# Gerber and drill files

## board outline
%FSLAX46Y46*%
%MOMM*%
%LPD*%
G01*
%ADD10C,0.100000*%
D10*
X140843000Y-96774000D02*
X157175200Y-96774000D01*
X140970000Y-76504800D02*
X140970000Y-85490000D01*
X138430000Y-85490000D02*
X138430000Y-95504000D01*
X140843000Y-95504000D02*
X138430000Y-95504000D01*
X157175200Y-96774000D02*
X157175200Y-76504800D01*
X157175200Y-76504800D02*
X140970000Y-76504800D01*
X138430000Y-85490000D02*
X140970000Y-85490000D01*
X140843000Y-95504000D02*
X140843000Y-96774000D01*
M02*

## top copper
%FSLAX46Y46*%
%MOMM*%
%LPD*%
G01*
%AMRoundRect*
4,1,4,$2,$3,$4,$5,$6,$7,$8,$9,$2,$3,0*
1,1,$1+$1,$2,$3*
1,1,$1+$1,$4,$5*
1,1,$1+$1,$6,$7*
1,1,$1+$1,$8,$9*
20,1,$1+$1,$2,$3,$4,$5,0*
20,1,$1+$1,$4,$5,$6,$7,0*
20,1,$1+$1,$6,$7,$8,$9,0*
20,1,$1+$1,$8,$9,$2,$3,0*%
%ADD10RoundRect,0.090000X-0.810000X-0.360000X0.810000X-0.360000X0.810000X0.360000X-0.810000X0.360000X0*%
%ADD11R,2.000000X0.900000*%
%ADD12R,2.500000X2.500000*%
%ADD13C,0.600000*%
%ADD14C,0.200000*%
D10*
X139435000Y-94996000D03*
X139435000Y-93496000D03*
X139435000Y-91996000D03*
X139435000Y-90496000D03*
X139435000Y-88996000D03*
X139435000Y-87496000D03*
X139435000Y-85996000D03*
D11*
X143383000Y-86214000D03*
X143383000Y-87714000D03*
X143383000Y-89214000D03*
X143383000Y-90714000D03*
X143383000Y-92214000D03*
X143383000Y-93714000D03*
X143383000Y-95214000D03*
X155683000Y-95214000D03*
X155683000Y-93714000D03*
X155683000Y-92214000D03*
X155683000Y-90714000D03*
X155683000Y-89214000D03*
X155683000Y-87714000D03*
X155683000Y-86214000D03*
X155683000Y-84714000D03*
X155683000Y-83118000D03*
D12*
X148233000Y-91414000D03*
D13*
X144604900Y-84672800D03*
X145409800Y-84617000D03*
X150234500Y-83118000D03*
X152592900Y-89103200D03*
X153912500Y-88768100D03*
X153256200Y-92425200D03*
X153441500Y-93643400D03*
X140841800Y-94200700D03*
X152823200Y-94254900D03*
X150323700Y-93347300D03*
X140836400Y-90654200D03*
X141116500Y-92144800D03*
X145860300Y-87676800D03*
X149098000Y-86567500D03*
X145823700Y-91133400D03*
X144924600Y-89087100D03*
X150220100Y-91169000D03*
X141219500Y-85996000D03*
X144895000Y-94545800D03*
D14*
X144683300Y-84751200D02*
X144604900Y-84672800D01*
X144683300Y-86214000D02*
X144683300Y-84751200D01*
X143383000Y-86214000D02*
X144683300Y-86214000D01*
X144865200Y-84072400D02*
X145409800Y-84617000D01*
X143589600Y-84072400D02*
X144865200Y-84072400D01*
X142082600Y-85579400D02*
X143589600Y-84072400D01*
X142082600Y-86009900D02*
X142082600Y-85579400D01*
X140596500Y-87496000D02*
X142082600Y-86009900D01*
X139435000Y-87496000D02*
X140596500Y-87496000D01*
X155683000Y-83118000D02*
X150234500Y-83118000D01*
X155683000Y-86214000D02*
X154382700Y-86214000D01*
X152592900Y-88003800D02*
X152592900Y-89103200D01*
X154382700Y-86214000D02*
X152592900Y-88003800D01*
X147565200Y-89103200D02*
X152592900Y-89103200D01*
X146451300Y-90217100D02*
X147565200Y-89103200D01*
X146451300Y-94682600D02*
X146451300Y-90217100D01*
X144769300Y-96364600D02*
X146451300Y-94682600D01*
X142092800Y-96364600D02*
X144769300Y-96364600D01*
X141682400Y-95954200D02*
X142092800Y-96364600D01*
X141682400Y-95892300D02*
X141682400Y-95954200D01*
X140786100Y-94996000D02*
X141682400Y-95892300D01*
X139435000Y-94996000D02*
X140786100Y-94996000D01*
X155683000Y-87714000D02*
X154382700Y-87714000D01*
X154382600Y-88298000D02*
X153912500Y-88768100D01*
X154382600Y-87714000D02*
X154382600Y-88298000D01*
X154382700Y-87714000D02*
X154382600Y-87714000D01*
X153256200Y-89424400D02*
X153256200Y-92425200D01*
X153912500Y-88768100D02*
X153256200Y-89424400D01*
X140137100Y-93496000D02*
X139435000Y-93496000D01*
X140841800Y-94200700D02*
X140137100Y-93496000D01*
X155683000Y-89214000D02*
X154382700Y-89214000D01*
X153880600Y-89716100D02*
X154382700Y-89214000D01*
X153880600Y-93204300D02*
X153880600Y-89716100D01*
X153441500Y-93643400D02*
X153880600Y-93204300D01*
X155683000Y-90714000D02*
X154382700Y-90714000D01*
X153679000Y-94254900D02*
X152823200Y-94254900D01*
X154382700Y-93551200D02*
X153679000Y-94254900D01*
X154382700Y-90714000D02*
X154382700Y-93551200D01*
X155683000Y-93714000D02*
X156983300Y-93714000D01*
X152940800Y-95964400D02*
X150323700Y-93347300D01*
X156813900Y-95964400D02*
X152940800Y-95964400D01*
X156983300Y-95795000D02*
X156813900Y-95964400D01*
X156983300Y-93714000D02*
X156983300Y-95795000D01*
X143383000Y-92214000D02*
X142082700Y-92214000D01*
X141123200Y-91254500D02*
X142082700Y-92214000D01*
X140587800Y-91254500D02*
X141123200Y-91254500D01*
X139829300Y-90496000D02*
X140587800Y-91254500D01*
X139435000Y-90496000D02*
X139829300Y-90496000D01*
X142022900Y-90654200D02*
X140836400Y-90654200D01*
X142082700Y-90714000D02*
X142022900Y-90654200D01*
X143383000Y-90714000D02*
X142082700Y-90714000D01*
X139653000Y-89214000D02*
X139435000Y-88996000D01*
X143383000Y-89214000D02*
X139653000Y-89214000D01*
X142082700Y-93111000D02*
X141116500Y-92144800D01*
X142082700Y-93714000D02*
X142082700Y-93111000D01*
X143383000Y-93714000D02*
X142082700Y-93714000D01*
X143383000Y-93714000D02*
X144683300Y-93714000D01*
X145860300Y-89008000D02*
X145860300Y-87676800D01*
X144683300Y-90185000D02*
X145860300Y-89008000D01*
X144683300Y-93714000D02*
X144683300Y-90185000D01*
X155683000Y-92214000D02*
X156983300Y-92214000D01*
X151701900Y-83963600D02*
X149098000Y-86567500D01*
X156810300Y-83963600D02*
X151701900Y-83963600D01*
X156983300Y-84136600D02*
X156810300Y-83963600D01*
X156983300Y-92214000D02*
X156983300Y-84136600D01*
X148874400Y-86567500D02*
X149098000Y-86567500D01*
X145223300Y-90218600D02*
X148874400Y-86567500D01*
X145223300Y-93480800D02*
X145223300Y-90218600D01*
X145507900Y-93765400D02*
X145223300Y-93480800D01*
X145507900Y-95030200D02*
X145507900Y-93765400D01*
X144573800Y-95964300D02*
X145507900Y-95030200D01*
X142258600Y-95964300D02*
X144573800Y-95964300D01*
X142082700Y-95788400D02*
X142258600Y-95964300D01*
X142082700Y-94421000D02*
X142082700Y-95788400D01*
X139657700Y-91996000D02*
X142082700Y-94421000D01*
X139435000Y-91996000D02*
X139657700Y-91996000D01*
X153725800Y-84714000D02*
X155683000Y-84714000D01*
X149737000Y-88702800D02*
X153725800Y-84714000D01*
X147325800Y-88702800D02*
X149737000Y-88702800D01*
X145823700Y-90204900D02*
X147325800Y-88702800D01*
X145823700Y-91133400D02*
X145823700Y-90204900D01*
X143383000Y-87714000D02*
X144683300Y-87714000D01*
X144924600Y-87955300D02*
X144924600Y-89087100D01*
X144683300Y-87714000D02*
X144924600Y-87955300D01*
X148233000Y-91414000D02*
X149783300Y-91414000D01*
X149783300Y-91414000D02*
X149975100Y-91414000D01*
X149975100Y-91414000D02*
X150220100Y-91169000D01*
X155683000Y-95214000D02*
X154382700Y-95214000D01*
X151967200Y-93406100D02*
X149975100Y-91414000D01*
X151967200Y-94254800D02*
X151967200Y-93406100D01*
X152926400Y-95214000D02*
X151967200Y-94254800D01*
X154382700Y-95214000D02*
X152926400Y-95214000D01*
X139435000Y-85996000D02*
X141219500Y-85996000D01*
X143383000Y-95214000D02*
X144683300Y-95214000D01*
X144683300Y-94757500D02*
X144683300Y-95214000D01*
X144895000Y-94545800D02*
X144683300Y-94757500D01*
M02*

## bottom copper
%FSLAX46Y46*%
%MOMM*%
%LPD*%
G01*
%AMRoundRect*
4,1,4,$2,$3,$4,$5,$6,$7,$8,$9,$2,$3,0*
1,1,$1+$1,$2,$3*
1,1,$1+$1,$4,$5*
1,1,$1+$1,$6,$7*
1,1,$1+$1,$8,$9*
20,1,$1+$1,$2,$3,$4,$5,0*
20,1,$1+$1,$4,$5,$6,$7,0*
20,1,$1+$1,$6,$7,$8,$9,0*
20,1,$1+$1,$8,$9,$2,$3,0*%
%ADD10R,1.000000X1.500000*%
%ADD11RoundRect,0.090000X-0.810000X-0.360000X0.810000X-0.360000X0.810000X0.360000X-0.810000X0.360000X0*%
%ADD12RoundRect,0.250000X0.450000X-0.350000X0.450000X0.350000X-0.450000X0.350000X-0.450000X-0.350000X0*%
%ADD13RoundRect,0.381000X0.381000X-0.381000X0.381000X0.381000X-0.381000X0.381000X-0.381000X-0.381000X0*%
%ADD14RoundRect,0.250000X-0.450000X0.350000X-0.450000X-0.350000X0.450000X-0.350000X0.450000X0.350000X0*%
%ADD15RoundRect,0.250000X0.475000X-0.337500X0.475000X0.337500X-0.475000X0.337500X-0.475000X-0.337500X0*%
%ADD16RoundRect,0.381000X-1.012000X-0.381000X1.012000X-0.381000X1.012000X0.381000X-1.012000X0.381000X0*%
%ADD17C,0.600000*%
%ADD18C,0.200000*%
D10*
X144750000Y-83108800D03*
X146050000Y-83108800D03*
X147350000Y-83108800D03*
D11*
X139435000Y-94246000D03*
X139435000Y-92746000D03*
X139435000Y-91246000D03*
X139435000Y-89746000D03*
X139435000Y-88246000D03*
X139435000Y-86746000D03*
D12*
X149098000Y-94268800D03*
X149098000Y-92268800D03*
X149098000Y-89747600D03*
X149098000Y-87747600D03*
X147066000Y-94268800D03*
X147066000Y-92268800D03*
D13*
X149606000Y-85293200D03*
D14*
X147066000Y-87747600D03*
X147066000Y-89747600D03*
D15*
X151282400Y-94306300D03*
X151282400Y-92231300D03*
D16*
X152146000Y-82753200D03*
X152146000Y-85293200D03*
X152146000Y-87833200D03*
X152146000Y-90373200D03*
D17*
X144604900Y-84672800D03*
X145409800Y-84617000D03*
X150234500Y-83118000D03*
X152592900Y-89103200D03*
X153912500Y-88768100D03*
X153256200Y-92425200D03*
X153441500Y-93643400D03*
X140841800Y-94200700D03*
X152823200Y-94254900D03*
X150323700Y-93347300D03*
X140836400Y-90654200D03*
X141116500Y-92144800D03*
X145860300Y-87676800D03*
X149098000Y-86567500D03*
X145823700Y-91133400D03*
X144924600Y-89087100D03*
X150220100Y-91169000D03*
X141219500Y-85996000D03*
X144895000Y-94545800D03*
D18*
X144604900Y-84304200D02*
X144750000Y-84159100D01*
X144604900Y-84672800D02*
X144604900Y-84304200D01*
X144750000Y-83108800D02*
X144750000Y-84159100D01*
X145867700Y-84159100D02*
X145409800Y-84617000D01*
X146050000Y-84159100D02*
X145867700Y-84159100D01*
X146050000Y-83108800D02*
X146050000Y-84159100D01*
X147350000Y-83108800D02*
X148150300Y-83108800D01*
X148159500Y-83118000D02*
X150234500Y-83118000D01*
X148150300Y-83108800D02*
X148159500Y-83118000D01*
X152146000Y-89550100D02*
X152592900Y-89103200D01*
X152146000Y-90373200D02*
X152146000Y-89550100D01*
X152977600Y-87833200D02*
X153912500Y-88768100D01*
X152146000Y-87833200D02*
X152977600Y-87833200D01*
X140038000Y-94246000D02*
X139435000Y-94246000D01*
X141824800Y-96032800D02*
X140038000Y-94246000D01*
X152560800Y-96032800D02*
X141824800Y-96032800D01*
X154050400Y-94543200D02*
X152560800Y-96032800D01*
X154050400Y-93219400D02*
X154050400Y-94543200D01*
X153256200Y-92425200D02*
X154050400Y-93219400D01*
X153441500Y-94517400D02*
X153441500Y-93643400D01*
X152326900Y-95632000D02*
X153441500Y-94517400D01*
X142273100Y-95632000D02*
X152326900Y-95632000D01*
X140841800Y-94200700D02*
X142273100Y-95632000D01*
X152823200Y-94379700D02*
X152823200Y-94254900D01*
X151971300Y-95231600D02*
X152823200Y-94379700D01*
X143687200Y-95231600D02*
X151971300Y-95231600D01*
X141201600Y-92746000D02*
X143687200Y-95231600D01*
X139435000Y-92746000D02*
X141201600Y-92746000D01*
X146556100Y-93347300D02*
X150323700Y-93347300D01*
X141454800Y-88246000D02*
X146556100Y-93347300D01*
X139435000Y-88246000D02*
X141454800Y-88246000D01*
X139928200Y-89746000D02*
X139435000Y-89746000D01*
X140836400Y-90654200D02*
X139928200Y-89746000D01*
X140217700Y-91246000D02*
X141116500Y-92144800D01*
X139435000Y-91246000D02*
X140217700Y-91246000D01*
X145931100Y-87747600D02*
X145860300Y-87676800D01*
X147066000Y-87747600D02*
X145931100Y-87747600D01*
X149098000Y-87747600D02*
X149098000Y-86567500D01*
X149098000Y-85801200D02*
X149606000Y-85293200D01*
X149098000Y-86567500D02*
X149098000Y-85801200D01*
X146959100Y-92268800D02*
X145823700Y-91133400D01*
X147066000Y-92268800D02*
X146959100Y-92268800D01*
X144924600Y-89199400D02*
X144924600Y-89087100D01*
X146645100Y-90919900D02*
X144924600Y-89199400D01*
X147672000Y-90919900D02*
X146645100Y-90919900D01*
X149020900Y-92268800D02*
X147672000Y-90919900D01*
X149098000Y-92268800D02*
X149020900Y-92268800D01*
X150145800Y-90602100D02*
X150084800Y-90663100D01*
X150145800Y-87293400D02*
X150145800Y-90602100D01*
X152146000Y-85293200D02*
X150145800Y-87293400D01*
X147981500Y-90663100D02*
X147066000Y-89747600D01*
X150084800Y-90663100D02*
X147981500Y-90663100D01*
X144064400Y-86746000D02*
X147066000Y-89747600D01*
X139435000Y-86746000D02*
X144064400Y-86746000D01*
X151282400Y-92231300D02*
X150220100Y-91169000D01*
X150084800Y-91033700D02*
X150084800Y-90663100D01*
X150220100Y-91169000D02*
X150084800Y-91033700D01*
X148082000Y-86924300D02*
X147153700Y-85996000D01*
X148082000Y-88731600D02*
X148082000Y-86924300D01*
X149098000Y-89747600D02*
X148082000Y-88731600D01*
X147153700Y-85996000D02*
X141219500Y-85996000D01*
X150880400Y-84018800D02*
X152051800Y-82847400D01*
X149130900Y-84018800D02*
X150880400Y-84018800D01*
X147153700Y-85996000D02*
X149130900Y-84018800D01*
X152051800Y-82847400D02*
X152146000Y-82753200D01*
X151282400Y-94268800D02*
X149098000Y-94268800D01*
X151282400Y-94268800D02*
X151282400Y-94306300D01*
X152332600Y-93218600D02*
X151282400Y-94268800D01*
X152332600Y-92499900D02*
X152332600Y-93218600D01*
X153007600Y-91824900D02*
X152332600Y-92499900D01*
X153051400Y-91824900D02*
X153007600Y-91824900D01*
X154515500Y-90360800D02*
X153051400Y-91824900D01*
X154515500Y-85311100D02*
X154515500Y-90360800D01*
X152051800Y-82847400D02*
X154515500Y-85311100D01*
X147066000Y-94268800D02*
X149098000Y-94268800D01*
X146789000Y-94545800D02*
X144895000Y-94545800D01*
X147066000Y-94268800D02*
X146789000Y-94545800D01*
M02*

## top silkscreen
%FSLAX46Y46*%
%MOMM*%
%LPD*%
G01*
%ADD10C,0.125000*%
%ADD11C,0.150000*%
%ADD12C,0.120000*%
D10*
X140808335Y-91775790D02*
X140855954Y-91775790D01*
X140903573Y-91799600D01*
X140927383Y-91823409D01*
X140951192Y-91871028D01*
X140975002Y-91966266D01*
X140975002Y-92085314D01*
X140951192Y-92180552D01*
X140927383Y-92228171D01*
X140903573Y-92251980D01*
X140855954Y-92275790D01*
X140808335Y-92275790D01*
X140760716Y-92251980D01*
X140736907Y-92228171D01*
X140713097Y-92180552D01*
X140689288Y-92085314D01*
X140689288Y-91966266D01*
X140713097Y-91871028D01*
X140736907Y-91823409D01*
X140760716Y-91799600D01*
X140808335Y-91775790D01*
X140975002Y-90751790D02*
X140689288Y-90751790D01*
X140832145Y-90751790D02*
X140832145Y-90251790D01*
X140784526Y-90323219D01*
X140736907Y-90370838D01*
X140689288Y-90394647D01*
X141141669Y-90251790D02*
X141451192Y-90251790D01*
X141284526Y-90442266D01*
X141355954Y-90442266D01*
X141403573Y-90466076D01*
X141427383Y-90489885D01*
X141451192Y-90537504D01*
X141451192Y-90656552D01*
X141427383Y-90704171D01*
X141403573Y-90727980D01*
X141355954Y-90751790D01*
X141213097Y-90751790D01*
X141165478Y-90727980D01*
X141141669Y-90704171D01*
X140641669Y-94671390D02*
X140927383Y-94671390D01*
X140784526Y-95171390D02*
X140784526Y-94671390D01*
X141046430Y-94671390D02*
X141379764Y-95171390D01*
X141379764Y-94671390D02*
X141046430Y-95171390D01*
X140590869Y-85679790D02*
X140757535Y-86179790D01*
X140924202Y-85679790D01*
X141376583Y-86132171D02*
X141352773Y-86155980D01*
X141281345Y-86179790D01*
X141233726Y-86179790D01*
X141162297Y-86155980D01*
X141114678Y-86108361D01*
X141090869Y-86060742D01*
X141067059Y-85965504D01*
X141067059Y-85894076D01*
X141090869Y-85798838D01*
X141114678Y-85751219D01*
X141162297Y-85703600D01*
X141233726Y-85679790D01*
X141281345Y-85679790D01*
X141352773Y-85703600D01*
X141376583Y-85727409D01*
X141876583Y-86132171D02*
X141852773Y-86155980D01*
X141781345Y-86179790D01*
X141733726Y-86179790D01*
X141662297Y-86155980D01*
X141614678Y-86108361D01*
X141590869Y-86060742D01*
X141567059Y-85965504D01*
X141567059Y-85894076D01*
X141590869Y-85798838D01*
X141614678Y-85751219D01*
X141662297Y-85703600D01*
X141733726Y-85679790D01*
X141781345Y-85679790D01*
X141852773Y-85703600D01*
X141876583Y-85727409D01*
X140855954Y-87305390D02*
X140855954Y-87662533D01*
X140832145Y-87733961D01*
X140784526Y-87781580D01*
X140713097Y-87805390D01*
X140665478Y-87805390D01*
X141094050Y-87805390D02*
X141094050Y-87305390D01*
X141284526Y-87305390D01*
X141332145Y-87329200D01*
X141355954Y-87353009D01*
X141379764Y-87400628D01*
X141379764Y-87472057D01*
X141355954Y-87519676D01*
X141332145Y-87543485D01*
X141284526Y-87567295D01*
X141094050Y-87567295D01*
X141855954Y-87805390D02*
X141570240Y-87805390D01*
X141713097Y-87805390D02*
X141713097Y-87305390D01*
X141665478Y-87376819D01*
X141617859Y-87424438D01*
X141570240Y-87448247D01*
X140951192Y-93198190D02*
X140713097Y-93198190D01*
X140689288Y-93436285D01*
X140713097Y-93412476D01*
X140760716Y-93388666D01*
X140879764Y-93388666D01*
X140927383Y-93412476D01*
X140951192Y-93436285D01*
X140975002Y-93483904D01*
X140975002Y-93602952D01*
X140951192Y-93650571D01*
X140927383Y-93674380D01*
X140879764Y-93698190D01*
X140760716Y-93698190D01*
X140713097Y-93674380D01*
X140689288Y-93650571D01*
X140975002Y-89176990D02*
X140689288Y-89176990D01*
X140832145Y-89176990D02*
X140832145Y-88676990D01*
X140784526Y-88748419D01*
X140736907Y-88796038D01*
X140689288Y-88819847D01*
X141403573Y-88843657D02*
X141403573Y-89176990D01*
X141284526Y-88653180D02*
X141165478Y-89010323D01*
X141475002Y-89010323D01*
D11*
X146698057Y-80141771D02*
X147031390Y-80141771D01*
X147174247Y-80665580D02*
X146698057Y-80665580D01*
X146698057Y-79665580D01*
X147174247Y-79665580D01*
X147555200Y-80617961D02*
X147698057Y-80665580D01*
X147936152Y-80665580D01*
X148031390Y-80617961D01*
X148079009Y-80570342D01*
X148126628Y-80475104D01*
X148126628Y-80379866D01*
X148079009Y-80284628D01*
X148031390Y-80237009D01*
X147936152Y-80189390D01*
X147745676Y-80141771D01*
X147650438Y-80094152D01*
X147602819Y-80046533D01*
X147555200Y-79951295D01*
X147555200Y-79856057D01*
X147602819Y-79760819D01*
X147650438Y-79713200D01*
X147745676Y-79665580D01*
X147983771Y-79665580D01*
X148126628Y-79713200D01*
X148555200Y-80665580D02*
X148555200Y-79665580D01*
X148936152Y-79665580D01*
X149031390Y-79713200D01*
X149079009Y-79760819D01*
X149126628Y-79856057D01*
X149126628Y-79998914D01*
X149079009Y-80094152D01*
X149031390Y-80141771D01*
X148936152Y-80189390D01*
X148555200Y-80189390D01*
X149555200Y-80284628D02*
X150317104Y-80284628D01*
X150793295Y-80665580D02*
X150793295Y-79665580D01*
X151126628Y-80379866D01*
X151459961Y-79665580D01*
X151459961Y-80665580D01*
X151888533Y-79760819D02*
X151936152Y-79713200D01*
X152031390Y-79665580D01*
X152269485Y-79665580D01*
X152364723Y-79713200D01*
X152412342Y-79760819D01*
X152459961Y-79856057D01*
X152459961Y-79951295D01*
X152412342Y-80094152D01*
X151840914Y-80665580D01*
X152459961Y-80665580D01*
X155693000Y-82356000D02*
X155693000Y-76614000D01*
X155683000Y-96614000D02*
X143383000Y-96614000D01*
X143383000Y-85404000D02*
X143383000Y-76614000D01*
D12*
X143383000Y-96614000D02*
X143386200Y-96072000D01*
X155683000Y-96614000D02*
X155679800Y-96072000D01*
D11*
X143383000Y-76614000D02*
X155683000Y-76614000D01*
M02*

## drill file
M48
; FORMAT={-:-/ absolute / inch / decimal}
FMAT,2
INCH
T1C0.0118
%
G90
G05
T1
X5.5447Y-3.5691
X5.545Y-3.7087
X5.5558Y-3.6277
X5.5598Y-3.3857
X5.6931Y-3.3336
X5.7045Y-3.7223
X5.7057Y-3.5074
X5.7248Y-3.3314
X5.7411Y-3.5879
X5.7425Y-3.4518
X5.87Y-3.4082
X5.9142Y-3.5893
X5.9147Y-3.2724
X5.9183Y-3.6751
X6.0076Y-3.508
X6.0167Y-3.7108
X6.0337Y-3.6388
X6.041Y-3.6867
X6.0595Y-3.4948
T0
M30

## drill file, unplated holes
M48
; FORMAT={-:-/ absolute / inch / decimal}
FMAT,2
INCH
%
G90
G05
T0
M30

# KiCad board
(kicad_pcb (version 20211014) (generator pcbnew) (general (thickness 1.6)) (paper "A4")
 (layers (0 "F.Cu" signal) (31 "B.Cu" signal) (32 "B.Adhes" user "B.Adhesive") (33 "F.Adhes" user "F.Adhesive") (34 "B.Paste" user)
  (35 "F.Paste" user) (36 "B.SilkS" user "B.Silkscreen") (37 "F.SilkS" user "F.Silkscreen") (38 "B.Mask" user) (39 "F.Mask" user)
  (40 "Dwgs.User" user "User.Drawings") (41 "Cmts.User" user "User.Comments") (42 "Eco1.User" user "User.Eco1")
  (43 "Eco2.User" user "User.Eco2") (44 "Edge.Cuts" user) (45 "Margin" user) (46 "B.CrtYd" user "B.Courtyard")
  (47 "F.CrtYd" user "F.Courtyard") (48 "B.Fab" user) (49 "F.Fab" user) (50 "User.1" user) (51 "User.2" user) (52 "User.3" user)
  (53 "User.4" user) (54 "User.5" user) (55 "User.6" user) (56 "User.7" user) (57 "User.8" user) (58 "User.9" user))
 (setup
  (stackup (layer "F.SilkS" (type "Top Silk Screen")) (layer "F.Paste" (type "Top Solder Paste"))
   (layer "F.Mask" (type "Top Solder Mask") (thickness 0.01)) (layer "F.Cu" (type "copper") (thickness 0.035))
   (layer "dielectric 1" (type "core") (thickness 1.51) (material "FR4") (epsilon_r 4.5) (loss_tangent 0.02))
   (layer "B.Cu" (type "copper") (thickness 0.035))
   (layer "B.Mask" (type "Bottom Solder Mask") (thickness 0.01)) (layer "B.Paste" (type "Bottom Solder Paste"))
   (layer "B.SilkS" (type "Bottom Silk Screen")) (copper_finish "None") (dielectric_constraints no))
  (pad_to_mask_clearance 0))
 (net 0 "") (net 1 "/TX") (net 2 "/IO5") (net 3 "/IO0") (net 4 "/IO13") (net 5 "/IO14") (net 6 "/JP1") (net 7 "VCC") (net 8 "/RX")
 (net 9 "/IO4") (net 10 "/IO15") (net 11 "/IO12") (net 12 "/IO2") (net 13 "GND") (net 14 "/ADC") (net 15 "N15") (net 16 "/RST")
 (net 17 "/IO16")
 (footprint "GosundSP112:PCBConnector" (layer "F.Cu") (at 140.335 94.996)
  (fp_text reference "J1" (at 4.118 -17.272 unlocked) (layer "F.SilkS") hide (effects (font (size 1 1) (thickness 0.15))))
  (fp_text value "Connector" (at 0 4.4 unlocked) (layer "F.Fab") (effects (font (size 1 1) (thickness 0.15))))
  (pad "1" smd roundrect (at -0.9 0) (size 1.8 0.9) (layers "F.Cu" "F.Paste" "F.Mask") (roundrect_rratio 0.1) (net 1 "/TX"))
  (pad "2" smd roundrect (at -0.9 -1.5) (size 1.8 0.9) (layers "F.Cu" "F.Paste" "F.Mask") (roundrect_rratio 0.1) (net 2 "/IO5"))
  (pad "3" smd roundrect (at -0.9 -3) (size 1.8 0.9) (layers "F.Cu" "F.Paste" "F.Mask") (roundrect_rratio 0.1) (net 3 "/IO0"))
  (pad "4" smd roundrect (at -0.9 -4.5) (size 1.8 0.9) (layers "F.Cu" "F.Paste" "F.Mask") (roundrect_rratio 0.1) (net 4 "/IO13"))
  (pad "5" smd roundrect (at -0.9 -6) (size 1.8 0.9) (layers "F.Cu" "F.Paste" "F.Mask") (roundrect_rratio 0.1) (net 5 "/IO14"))
  (pad "6" smd roundrect (at -0.9 -7.5) (size 1.8 0.9) (layers "F.Cu" "F.Paste" "F.Mask") (roundrect_rratio 0.1) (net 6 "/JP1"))
  (pad "7" smd roundrect (at -0.9 -9) (size 1.8 0.9) (layers "F.Cu" "F.Paste" "F.Mask") (roundrect_rratio 0.1) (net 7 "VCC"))
  (pad "8" smd roundrect (at -0.9 -0.75) (size 1.8 0.9) (layers "B.Cu" "B.Paste" "B.Mask") (roundrect_rratio 0.1) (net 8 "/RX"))
  (pad "9" smd roundrect (at -0.9 -2.25) (size 1.8 0.9) (layers "B.Cu" "B.Paste" "B.Mask") (roundrect_rratio 0.1) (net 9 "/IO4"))
  (pad "10" smd roundrect (at -0.9 -3.75) (size 1.8 0.9) (layers "B.Cu" "B.Paste" "B.Mask") (roundrect_rratio 0.1) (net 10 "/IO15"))
  (pad "11" smd roundrect (at -0.9 -5.25) (size 1.8 0.9) (layers "B.Cu" "B.Paste" "B.Mask") (roundrect_rratio 0.1) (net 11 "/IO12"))
  (pad "12" smd roundrect (at -0.9 -6.75) (size 1.8 0.9) (layers "B.Cu" "B.Paste" "B.Mask") (roundrect_rratio 0.1) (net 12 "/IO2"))
  (pad "13" smd roundrect (at -0.9 -8.25) (size 1.8 0.9) (layers "B.Cu" "B.Paste" "B.Mask") (roundrect_rratio 0.1) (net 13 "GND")))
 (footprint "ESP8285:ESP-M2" (layer "F.Cu") (at 149.533 89.214)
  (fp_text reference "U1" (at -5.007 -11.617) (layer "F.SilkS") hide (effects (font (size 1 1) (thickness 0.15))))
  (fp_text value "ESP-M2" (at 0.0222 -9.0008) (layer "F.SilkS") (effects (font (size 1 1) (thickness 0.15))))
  (fp_line (start 6.16 -6.858) (end 6.16 -12.6) (layer "F.SilkS") (width 0.15))
  (fp_line (start 6.15 7.4) (end -6.15 7.4) (layer "F.SilkS") (width 0.15))
  (fp_line (start -6.15 -3.81) (end -6.15 -12.6) (layer "F.SilkS") (width 0.15))
  (fp_line (start -6.15 7.4) (end -6.1468 6.858) (layer "F.SilkS") (width 0.12))
  (fp_line (start 6.15 7.4) (end 6.1468 6.858) (layer "F.SilkS") (width 0.12))
  (fp_line (start -6.15 -12.6) (end 6.15 -12.6) (layer "F.SilkS") (width 0.15))
  (pad "1" smd rect (at -6.15 -3 90) (size 0.9 2) (layers "F.Cu" "F.Paste" "F.Mask") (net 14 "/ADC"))
  (pad "2" smd rect (at -6.15 -1.5 90) (size 0.9 2) (layers "F.Cu" "F.Paste" "F.Mask") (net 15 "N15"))
  (pad "3" smd rect (at -6.15 0 90) (size 0.9 2) (layers "F.Cu" "F.Paste" "F.Mask") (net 5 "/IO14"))
  (pad "4" smd rect (at -6.15 1.5 90) (size 0.9 2) (layers "F.Cu" "F.Paste" "F.Mask") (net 11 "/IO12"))
  (pad "5" smd rect (at -6.15 3 90) (size 0.9 2) (layers "F.Cu" "F.Paste" "F.Mask") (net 4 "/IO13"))
  (pad "6" smd rect (at -6.15 4.5 90) (size 0.9 2) (layers "F.Cu" "F.Paste" "F.Mask") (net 10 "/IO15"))
  (pad "7" smd rect (at -6.15 6 90) (size 0.9 2) (layers "F.Cu" "F.Paste" "F.Mask") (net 7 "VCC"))
  (pad "8" smd rect (at 6.15 6 90) (size 0.9 2) (layers "F.Cu" "F.Paste" "F.Mask") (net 13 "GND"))
  (pad "9" smd rect (at 6.15 4.5 90) (size 0.9 2) (layers "F.Cu" "F.Paste" "F.Mask") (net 12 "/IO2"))
  (pad "10" smd rect (at 6.15 3 90) (size 0.9 2) (layers "F.Cu" "F.Paste" "F.Mask") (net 3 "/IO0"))
  (pad "11" smd rect (at 6.15 1.5 90) (size 0.9 2) (layers "F.Cu" "F.Paste" "F.Mask") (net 9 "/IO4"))
  (pad "12" smd rect (at 6.15 0 90) (size 0.9 2) (layers "F.Cu" "F.Paste" "F.Mask") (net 2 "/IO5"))
  (pad "13" smd rect (at 6.15 -1.5 90) (size 0.9 2) (layers "F.Cu" "F.Paste" "F.Mask") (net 8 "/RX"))
  (pad "14" smd rect (at 6.15 -3 90) (size 0.9 2) (layers "F.Cu" "F.Paste" "F.Mask") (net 1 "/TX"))
  (pad "15" smd rect (at 6.15 -4.5 90) (size 0.9 2) (layers "F.Cu" "F.Paste" "F.Mask") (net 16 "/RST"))
  (pad "16" smd rect (at 6.15 -6.096 90) (size 0.9 2) (layers "F.Cu" "F.Paste" "F.Mask") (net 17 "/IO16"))
  (pad "17" smd rect (at -1.3 2.2 90) (size 2.5 2.5) (layers "F.Cu" "F.Paste" "F.Mask") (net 13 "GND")))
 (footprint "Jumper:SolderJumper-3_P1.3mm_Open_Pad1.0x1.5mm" (layer "B.Cu") (at 146.05 83.1088)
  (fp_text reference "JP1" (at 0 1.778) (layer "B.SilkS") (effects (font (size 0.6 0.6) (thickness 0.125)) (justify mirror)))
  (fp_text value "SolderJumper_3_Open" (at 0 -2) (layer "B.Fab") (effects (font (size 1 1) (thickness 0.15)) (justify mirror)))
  (pad "1" smd rect (at -1.3 0) (size 1 1.5) (layers "B.Cu" "B.Mask") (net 14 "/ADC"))
  (pad "2" smd rect (at 0 0) (size 1 1.5) (layers "B.Cu" "B.Mask") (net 6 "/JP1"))
  (pad "3" smd rect (at 1.3 0) (size 1 1.5) (layers "B.Cu" "B.Mask") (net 17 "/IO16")))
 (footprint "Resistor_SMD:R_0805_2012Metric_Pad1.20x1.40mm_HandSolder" (layer "B.Cu") (at 149.098 93.2688 90)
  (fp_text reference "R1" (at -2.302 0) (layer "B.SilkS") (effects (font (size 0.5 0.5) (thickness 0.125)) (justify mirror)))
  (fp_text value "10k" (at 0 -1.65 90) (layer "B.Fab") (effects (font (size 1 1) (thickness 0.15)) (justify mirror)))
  (pad "1" smd roundrect (at -1 0 90) (size 1.2 1.4) (layers "B.Cu" "B.Paste" "B.Mask") (roundrect_rratio 0.2083333333) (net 7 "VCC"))
  (pad "2" smd roundrect (at 1 0 90) (size 1.2 1.4) (layers "B.Cu" "B.Paste" "B.Mask") (roundrect_rratio 0.2083333333) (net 15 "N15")))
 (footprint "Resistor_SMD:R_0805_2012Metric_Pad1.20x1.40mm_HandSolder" (layer "B.Cu") (at 149.098 88.7476 90)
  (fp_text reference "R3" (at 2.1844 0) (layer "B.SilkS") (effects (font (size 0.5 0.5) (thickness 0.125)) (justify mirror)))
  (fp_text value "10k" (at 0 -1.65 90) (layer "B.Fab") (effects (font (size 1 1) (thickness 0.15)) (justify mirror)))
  (pad "1" smd roundrect (at -1 0 90) (size 1.2 1.4) (layers "B.Cu" "B.Paste" "B.Mask") (roundrect_rratio 0.2083333333) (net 7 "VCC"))
  (pad "2" smd roundrect (at 1 0 90) (size 1.2 1.4) (layers "B.Cu" "B.Paste" "B.Mask") (roundrect_rratio 0.2083333333) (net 3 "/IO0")))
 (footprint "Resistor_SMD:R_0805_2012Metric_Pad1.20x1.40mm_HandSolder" (layer "B.Cu") (at 147.066 93.2688 90)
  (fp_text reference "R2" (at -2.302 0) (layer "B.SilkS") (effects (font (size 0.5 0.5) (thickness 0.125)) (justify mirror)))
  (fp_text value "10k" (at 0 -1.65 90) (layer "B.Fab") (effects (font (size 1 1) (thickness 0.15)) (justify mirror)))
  (pad "1" smd roundrect (at -1 0 90) (size 1.2 1.4) (layers "B.Cu" "B.Paste" "B.Mask") (roundrect_rratio 0.2083333333) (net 7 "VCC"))
  (pad "2" smd roundrect (at 1 0 90) (size 1.2 1.4) (layers "B.Cu" "B.Paste" "B.Mask") (roundrect_rratio 0.2083333333) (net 16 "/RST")))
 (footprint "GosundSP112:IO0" (layer "B.Cu") (at 147.066 85.2932 90)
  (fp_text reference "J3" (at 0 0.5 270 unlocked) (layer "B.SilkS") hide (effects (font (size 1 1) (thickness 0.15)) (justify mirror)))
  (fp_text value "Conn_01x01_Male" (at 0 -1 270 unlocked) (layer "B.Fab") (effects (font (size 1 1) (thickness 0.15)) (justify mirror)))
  (pad "1" smd roundrect (at 0 2.54 90) (size 1.524 1.524) (layers "B.Cu" "B.Paste" "B.Mask") (roundrect_rratio 0.25) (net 3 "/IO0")))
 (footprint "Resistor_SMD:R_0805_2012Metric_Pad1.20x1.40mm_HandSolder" (layer "B.Cu") (at 147.066 88.7476 -90)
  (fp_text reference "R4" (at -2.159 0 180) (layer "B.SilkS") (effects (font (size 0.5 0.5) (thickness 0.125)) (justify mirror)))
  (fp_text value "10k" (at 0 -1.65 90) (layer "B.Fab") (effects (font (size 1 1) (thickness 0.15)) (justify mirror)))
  (pad "1" smd roundrect (at -1 0 270) (size 1.2 1.4) (layers "B.Cu" "B.Paste" "B.Mask") (roundrect_rratio 0.2083333333) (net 10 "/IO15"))
  (pad "2" smd roundrect (at 1 0 270) (size 1.2 1.4) (layers "B.Cu" "B.Paste" "B.Mask") (roundrect_rratio 0.2083333333) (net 13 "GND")))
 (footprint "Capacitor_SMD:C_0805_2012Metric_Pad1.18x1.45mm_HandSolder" (layer "B.Cu") (at 151.2824 93.2688 90)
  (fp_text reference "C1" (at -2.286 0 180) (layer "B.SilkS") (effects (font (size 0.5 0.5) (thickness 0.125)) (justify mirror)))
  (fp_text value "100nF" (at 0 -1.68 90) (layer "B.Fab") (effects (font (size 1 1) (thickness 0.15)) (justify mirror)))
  (pad "1" smd roundrect (at -1.0375 0 90) (size 1.175 1.45) (layers "B.Cu" "B.Paste" "B.Mask") (roundrect_rratio 0.2127659574)
   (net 7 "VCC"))
  (pad "2" smd roundrect (at 1.0375 0 90) (size 1.175 1.45) (layers "B.Cu" "B.Paste" "B.Mask") (roundrect_rratio 0.2127659574)
   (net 13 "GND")))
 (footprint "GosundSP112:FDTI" (layer "B.Cu") (at 152.146 82.7532)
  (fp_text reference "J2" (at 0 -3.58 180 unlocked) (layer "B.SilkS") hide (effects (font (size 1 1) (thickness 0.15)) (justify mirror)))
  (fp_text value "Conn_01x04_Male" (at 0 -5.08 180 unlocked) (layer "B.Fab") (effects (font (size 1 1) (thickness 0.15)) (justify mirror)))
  (pad "1" smd roundrect (at 0 0) (size 2.786 1.524) (layers "B.Cu" "B.Paste" "B.Mask") (roundrect_rratio 0.25) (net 7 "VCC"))
  (pad "2" smd roundrect (at 0 2.54) (size 2.786 1.524) (layers "B.Cu" "B.Paste" "B.Mask") (roundrect_rratio 0.25) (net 13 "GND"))
  (pad "3" smd roundrect (at 0 5.08) (size 2.786 1.524) (layers "B.Cu" "B.Paste" "B.Mask") (roundrect_rratio 0.25) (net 8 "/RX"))
  (pad "4" smd roundrect (at 0 7.62) (size 2.786 1.524) (layers "B.Cu" "B.Paste" "B.Mask") (roundrect_rratio 0.25) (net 1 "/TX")))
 (gr_line (start 140.843 96.774) (end 157.1752 96.774) (layer "Edge.Cuts") (width 0.1))
 (gr_line (start 140.97 76.5048) (end 140.97 85.49) (layer "Edge.Cuts") (width 0.1))
 (gr_line (start 138.43 85.49) (end 138.43 95.504) (layer "Edge.Cuts") (width 0.1))
 (gr_line (start 140.843 95.504) (end 138.43 95.504) (layer "Edge.Cuts") (width 0.1))
 (gr_line (start 157.1752 96.774) (end 157.1752 76.5048) (layer "Edge.Cuts") (width 0.1))
 (gr_line (start 157.1752 76.5048) (end 140.97 76.5048) (layer "Edge.Cuts") (width 0.1))
 (gr_line (start 138.43 85.49) (end 140.97 85.49) (layer "Edge.Cuts") (width 0.1))
 (gr_line (start 140.843 95.504) (end 140.843 96.774) (layer "Edge.Cuts") (width 0.1))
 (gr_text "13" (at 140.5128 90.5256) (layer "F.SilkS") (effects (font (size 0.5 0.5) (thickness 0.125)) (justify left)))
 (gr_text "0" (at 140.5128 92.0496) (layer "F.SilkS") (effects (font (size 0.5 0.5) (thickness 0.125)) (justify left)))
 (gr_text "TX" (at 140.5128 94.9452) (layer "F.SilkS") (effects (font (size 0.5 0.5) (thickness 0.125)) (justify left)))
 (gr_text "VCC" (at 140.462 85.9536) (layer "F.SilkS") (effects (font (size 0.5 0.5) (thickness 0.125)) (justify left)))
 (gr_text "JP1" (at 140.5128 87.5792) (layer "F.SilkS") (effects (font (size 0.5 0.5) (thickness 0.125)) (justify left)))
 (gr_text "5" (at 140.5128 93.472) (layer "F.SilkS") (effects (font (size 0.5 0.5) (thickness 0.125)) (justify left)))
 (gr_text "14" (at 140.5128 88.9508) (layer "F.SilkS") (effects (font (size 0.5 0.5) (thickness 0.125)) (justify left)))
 (segment (start 144.6833 94.7575) (end 144.6833 95.214) (width 0.2) (layer "F.Cu") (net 7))
 (segment (start 143.383 95.214) (end 144.6833 95.214) (width 0.2) (layer "F.Cu") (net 7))
 (segment (start 144.895 94.5458) (end 144.6833 94.7575) (width 0.2) (layer "F.Cu") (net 7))
 (segment (start 139.435 85.996) (end 141.2195 85.996) (width 0.2) (layer "F.Cu") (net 7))
 (via (at 144.895 94.5458) (size 0.6) (drill 0.3) (layers "F.Cu" "B.Cu") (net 7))
 (via (at 141.2195 85.996) (size 0.6) (drill 0.3) (layers "F.Cu" "B.Cu") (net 7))
 (segment (start 152.3326 92.4999) (end 152.3326 93.2186) (width 0.2) (layer "B.Cu") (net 7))
 (segment (start 150.8804 84.0188) (end 152.0518 82.8474) (width 0.2) (layer "B.Cu") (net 7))
 (segment (start 147.066 94.2688) (end 149.098 94.2688) (width 0.2) (layer "B.Cu") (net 7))
 (segment (start 153.0514 91.8249) (end 153.0076 91.8249) (width 0.2) (layer "B.Cu") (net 7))
 (segment (start 147.1537 85.996) (end 141.2195 85.996) (width 0.2) (layer "B.Cu") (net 7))
 (segment (start 151.2824 94.2688) (end 149.098 94.2688) (width 0.2) (layer "B.Cu") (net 7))
 (segment (start 148.082 88.7316) (end 148.082 86.9243) (width 0.2) (layer "B.Cu") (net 7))
 (segment (start 146.789 94.5458) (end 144.895 94.5458) (width 0.2) (layer "B.Cu") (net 7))
 (segment (start 147.066 94.2688) (end 146.789 94.5458) (width 0.2) (layer "B.Cu") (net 7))
 (segment (start 152.0518 82.8474) (end 154.5155 85.3111) (width 0.2) (layer "B.Cu") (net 7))
 (segment (start 152.3326 93.2186) (end 151.2824 94.2688) (width 0.2) (layer "B.Cu") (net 7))
 (segment (start 153.0076 91.8249) (end 152.3326 92.4999) (width 0.2) (layer "B.Cu") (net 7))
 (segment (start 148.082 86.9243) (end 147.1537 85.996) (width 0.2) (layer "B.Cu") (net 7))
 (segment (start 147.1537 85.996) (end 149.1309 84.0188) (width 0.2) (layer "B.Cu") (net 7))
 (segment (start 149.1309 84.0188) (end 150.8804 84.0188) (width 0.2) (layer "B.Cu") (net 7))
 (segment (start 149.098 89.7476) (end 148.082 88.7316) (width 0.2) (layer "B.Cu") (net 7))
 (segment (start 152.0518 82.8474) (end 152.146 82.7532) (width 0.2) (layer "B.Cu") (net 7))
 (segment (start 151.2824 94.2688) (end 151.2824 94.3063) (width 0.2) (layer "B.Cu") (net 7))
 (segment (start 154.5155 85.3111) (end 154.5155 90.3608) (width 0.2) (layer "B.Cu") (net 7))
 (segment (start 154.5155 90.3608) (end 153.0514 91.8249) (width 0.2) (layer "B.Cu") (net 7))
 (segment (start 149.7833 91.414) (end 149.9751 91.414) (width 0.2) (layer "F.Cu") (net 13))
 (segment (start 149.9751 91.414) (end 150.2201 91.169) (width 0.2) (layer "F.Cu") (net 13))
 (segment (start 154.3827 95.214) (end 152.9264 95.214) (width 0.2) (layer "F.Cu") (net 13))
 (segment (start 152.9264 95.214) (end 151.9672 94.2548) (width 0.2) (layer "F.Cu") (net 13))
 (segment (start 151.9672 94.2548) (end 151.9672 93.4061) (width 0.2) (layer "F.Cu") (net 13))
 (segment (start 155.683 95.214) (end 154.3827 95.214) (width 0.2) (layer "F.Cu") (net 13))
 (segment (start 151.9672 93.4061) (end 149.9751 91.414) (width 0.2) (layer "F.Cu") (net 13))
 (segment (start 148.233 91.414) (end 149.7833 91.414) (width 0.2) (layer "F.Cu") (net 13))
 (via (at 150.2201 91.169) (size 0.6) (drill 0.3) (layers "F.Cu" "B.Cu") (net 13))
 (segment (start 150.0848 91.0337) (end 150.0848 90.6631) (width 0.2) (layer "B.Cu") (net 13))
 (segment (start 150.0848 90.6631) (end 147.9815 90.6631) (width 0.2) (layer "B.Cu") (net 13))
 (segment (start 144.0644 86.746) (end 147.066 89.7476) (width 0.2) (layer "B.Cu") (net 13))
 (segment (start 150.1458 87.2934) (end 150.1458 90.6021) (width 0.2) (layer "B.Cu") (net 13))
 (segment (start 147.9815 90.6631) (end 147.066 89.7476) (width 0.2) (layer "B.Cu") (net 13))
 (segment (start 150.2201 91.169) (end 150.0848 91.0337) (width 0.2) (layer "B.Cu") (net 13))
 (segment (start 152.146 85.2932) (end 150.1458 87.2934) (width 0.2) (layer "B.Cu") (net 13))
 (segment (start 151.2824 92.2313) (end 150.2201 91.169) (width 0.2) (layer "B.Cu") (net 13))
 (segment (start 139.435 86.746) (end 144.0644 86.746) (width 0.2) (layer "B.Cu") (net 13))
 (segment (start 150.1458 90.6021) (end 150.0848 90.6631) (width 0.2) (layer "B.Cu") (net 13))
 (segment (start 144.6833 87.714) (end 144.9246 87.9553) (width 0.2) (layer "F.Cu") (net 15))
 (segment (start 143.383 87.714) (end 144.6833 87.714) (width 0.2) (layer "F.Cu") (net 15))
 (segment (start 144.9246 87.9553) (end 144.9246 89.0871) (width 0.2) (layer "F.Cu") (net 15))
 (via (at 144.9246 89.0871) (size 0.6) (drill 0.3) (layers "F.Cu" "B.Cu") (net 15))
 (segment (start 147.672 90.9199) (end 146.6451 90.9199) (width 0.2) (layer "B.Cu") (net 15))
 (segment (start 149.098 92.2688) (end 149.0209 92.2688) (width 0.2) (layer "B.Cu") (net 15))
 (segment (start 149.0209 92.2688) (end 147.672 90.9199) (width 0.2) (layer "B.Cu") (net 15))
 (segment (start 146.6451 90.9199) (end 144.9246 89.1994) (width 0.2) (layer "B.Cu") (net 15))
 (segment (start 144.9246 89.1994) (end 144.9246 89.0871) (width 0.2) (layer "B.Cu") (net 15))
 (segment (start 145.8237 91.1334) (end 145.8237 90.2049) (width 0.2) (layer "F.Cu") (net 16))
 (segment (start 147.3258 88.7028) (end 149.737 88.7028) (width 0.2) (layer "F.Cu") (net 16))
 (segment (start 145.8237 90.2049) (end 147.3258 88.7028) (width 0.2) (layer "F.Cu") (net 16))
 (segment (start 153.7258 84.714) (end 155.683 84.714) (width 0.2) (layer "F.Cu") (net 16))
 (segment (start 149.737 88.7028) (end 153.7258 84.714) (width 0.2) (layer "F.Cu") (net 16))
 (via (at 145.8237 91.1334) (size 0.6) (drill 0.3) (layers "F.Cu" "B.Cu") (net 16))
 (segment (start 147.066 92.2688) (end 146.9591 92.2688) (width 0.2) (layer "B.Cu") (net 16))
 (segment (start 146.9591 92.2688) (end 145.8237 91.1334) (width 0.2) (layer "B.Cu") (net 16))
 (segment (start 156.9833 84.1366) (end 156.8103 83.9636) (width 0.2) (layer "F.Cu") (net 3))
 (segment (start 142.0827 95.7884) (end 142.2586 95.9643) (width 0.2) (layer "F.Cu") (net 3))
 (segment (start 145.2233 90.2186) (end 148.8744 86.5675) (width 0.2) (layer "F.Cu") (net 3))
 (segment (start 151.7019 83.9636) (end 149.098 86.5675) (width 0.2) (layer "F.Cu") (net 3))
 (segment (start 145.2233 93.4808) (end 145.2233 90.2186) (width 0.2) (layer "F.Cu") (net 3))
 (segment (start 156.9833 92.214) (end 156.9833 84.1366) (width 0.2) (layer "F.Cu") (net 3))
 (segment (start 155.683 92.214) (end 156.9833 92.214) (width 0.2) (layer "F.Cu") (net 3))
 (segment (start 142.0827 94.421) (end 142.0827 95.7884) (width 0.2) (layer "F.Cu") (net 3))
 (segment (start 142.2586 95.9643) (end 144.5738 95.9643) (width 0.2) (layer "F.Cu") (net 3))
 (segment (start 148.8744 86.5675) (end 149.098 86.5675) (width 0.2) (layer "F.Cu") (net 3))
 (segment (start 139.435 91.996) (end 139.6577 91.996) (width 0.2) (layer "F.Cu") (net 3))
 (segment (start 139.6577 91.996) (end 142.0827 94.421) (width 0.2) (layer "F.Cu") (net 3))
 (segment (start 145.5079 95.0302) (end 145.5079 93.7654) (width 0.2) (layer "F.Cu") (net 3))
 (segment (start 145.5079 93.7654) (end 145.2233 93.4808) (width 0.2) (layer "F.Cu") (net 3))
 (segment (start 156.8103 83.9636) (end 151.7019 83.9636) (width 0.2) (layer "F.Cu") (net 3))
 (segment (start 144.5738 95.9643) (end 145.5079 95.0302) (width 0.2) (layer "F.Cu") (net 3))
 (via (at 149.098 86.5675) (size 0.6) (drill 0.3) (layers "F.Cu" "B.Cu") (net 3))
 (segment (start 149.098 87.7476) (end 149.098 86.5675) (width 0.2) (layer "B.Cu") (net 3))
 (segment (start 149.098 86.5675) (end 149.098 85.8012) (width 0.2) (layer "B.Cu") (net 3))
 (segment (start 149.098 85.8012) (end 149.606 85.2932) (width 0.2) (layer "B.Cu") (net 3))
 (segment (start 144.6833 90.185) (end 145.8603 89.008) (width 0.2) (layer "F.Cu") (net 10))
 (segment (start 143.383 93.714) (end 142.0827 93.714) (width 0.2) (layer "F.Cu") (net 10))
 (segment (start 144.6833 93.714) (end 144.6833 90.185) (width 0.2) (layer "F.Cu") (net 10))
 (segment (start 142.0827 93.714) (end 142.0827 93.111) (width 0.2) (layer "F.Cu") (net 10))
 (segment (start 142.0827 93.111) (end 141.1165 92.1448) (width 0.2) (layer "F.Cu") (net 10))
 (segment (start 145.8603 89.008) (end 145.8603 87.6768) (width 0.2) (layer "F.Cu") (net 10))
 (segment (start 143.383 93.714) (end 144.6833 93.714) (width 0.2) (layer "F.Cu") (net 10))
 (via (at 145.8603 87.6768) (size 0.6) (drill 0.3) (layers "F.Cu" "B.Cu") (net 10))
 (via (at 141.1165 92.1448) (size 0.6) (drill 0.3) (layers "F.Cu" "B.Cu") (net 10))
 (segment (start 139.435 91.246) (end 140.2177 91.246) (width 0.2) (layer "B.Cu") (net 10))
 (segment (start 140.2177 91.246) (end 141.1165 92.1448) (width 0.2) (layer "B.Cu") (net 10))
 (segment (start 145.9311 87.7476) (end 145.8603 87.6768) (width 0.2) (layer "B.Cu") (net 10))
 (segment (start 147.066 87.7476) (end 145.9311 87.7476) (width 0.2) (layer "B.Cu") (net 10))
 (segment (start 143.383 89.214) (end 139.653 89.214) (width 0.2) (layer "F.Cu") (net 5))
 (segment (start 139.653 89.214) (end 139.435 88.996) (width 0.2) (layer "F.Cu") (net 5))
 (segment (start 143.383 90.714) (end 142.0827 90.714) (width 0.2) (layer "F.Cu") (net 11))
 (segment (start 142.0827 90.714) (end 142.0229 90.6542) (width 0.2) (layer "F.Cu") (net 11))
 (segment (start 142.0229 90.6542) (end 140.8364 90.6542) (width 0.2) (layer "F.Cu") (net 11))
 (via (at 140.8364 90.6542) (size 0.6) (drill 0.3) (layers "F.Cu" "B.Cu") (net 11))
 (segment (start 139.9282 89.746) (end 139.435 89.746) (width 0.2) (layer "B.Cu") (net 11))
 (segment (start 140.8364 90.6542) (end 139.9282 89.746) (width 0.2) (layer "B.Cu") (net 11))
 (segment (start 139.8293 90.496) (end 140.5878 91.2545) (width 0.2) (layer "F.Cu") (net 4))
 (segment (start 143.383 92.214) (end 142.0827 92.214) (width 0.2) (layer "F.Cu") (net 4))
 (segment (start 141.1232 91.2545) (end 142.0827 92.214) (width 0.2) (layer "F.Cu") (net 4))
 (segment (start 140.5878 91.2545) (end 141.1232 91.2545) (width 0.2) (layer "F.Cu") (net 4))
 (segment (start 139.435 90.496) (end 139.8293 90.496) (width 0.2) (layer "F.Cu") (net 4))
 (segment (start 155.683 93.714) (end 156.9833 93.714) (width 0.2) (layer "F.Cu") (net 12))
 (segment (start 152.9408 95.9644) (end 150.3237 93.3473) (width 0.2) (layer "F.Cu") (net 12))
 (segment (start 156.9833 95.795) (end 156.8139 95.9644) (width 0.2) (layer "F.Cu") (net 12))
 (segment (start 156.9833 93.714) (end 156.9833 95.795) (width 0.2) (layer "F.Cu") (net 12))
 (segment (start 156.8139 95.9644) (end 152.9408 95.9644) (width 0.2) (layer "F.Cu") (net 12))
 (via (at 150.3237 93.3473) (size 0.6) (drill 0.3) (layers "F.Cu" "B.Cu") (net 12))
 (segment (start 139.435 88.246) (end 141.4548 88.246) (width 0.2) (layer "B.Cu") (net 12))
 (segment (start 146.5561 93.3473) (end 150.3237 93.3473) (width 0.2) (layer "B.Cu") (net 12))
 (segment (start 141.4548 88.246) (end 146.5561 93.3473) (width 0.2) (layer "B.Cu") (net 12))
 (segment (start 153.679 94.2549) (end 152.8232 94.2549) (width 0.2) (layer "F.Cu") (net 9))
 (segment (start 154.3827 90.714) (end 154.3827 93.5512) (width 0.2) (layer "F.Cu") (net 9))
 (segment (start 155.683 90.714) (end 154.3827 90.714) (width 0.2) (layer "F.Cu") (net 9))
 (segment (start 154.3827 93.5512) (end 153.679 94.2549) (width 0.2) (layer "F.Cu") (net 9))
 (via (at 152.8232 94.2549) (size 0.6) (drill 0.3) (layers "F.Cu" "B.Cu") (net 9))
 (segment (start 151.9713 95.2316) (end 152.8232 94.3797) (width 0.2) (layer "B.Cu") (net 9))
 (segment (start 152.8232 94.3797) (end 152.8232 94.2549) (width 0.2) (layer "B.Cu") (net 9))
 (segment (start 143.6872 95.2316) (end 151.9713 95.2316) (width 0.2) (layer "B.Cu") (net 9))
 (segment (start 141.2016 92.746) (end 143.6872 95.2316) (width 0.2) (layer "B.Cu") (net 9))
 (segment (start 139.435 92.746) (end 141.2016 92.746) (width 0.2) (layer "B.Cu") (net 9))
 (segment (start 155.683 89.214) (end 154.3827 89.214) (width 0.2) (layer "F.Cu") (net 2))
 (segment (start 153.8806 93.2043) (end 153.8806 89.7161) (width 0.2) (layer "F.Cu") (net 2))
 (segment (start 153.8806 89.7161) (end 154.3827 89.214) (width 0.2) (layer "F.Cu") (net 2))
 (segment (start 153.4415 93.6434) (end 153.8806 93.2043) (width 0.2) (layer "F.Cu") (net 2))
 (segment (start 140.1371 93.496) (end 139.435 93.496) (width 0.2) (layer "F.Cu") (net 2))
 (segment (start 140.8418 94.2007) (end 140.1371 93.496) (width 0.2) (layer "F.Cu") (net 2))
 (via (at 153.4415 93.6434) (size 0.6) (drill 0.3) (layers "F.Cu" "B.Cu") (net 2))
 (via (at 140.8418 94.2007) (size 0.6) (drill 0.3) (layers "F.Cu" "B.Cu") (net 2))
 (segment (start 152.3269 95.632) (end 153.4415 94.5174) (width 0.2) (layer "B.Cu") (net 2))
 (segment (start 142.2731 95.632) (end 152.3269 95.632) (width 0.2) (layer "B.Cu") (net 2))
 (segment (start 153.4415 94.5174) (end 153.4415 93.6434) (width 0.2) (layer "B.Cu") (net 2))
 (segment (start 140.8418 94.2007) (end 142.2731 95.632) (width 0.2) (layer "B.Cu") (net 2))
 (segment (start 153.9125 88.7681) (end 153.2562 89.4244) (width 0.2) (layer "F.Cu") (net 8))
 (segment (start 154.3826 87.714) (end 154.3826 88.298) (width 0.2) (layer "F.Cu") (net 8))
 (segment (start 154.3827 87.714) (end 154.3826 87.714) (width 0.2) (layer "F.Cu") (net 8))
 (segment (start 155.683 87.714) (end 154.3827 87.714) (width 0.2) (layer "F.Cu") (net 8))
 (segment (start 153.2562 89.4244) (end 153.2562 92.4252) (width 0.2) (layer "F.Cu") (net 8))
 (segment (start 154.3826 88.298) (end 153.9125 88.7681) (width 0.2) (layer "F.Cu") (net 8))
 (via (at 153.9125 88.7681) (size 0.6) (drill 0.3) (layers "F.Cu" "B.Cu") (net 8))
 (via (at 153.2562 92.4252) (size 0.6) (drill 0.3) (layers "F.Cu" "B.Cu") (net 8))
 (segment (start 152.9776 87.8332) (end 153.9125 88.7681) (width 0.2) (layer "B.Cu") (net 8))
 (segment (start 141.8248 96.0328) (end 140.038 94.246) (width 0.2) (layer "B.Cu") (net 8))
 (segment (start 152.146 87.8332) (end 152.9776 87.8332) (width 0.2) (layer "B.Cu") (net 8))
 (segment (start 153.2562 92.4252) (end 154.0504 93.2194) (width 0.2) (layer "B.Cu") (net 8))
 (segment (start 154.0504 93.2194) (end 154.0504 94.5432) (width 0.2) (layer "B.Cu") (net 8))
 (segment (start 152.5608 96.0328) (end 141.8248 96.0328) (width 0.2) (layer "B.Cu") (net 8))
 (segment (start 154.0504 94.5432) (end 152.5608 96.0328) (width 0.2) (layer "B.Cu") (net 8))
 (segment (start 140.038 94.246) (end 139.435 94.246) (width 0.2) (layer "B.Cu") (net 8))
 (segment (start 152.5929 88.0038) (end 152.5929 89.1032) (width 0.2) (layer "F.Cu") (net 1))
 (segment (start 139.435 94.996) (end 140.7861 94.996) (width 0.2) (layer "F.Cu") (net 1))
 (segment (start 144.7693 96.3646) (end 146.4513 94.6826) (width 0.2) (layer "F.Cu") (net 1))
 (segment (start 140.7861 94.996) (end 141.6824 95.8923) (width 0.2) (layer "F.Cu") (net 1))
 (segment (start 142.0928 96.3646) (end 144.7693 96.3646) (width 0.2) (layer "F.Cu") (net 1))
 (segment (start 155.683 86.214) (end 154.3827 86.214) (width 0.2) (layer "F.Cu") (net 1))
 (segment (start 141.6824 95.9542) (end 142.0928 96.3646) (width 0.2) (layer "F.Cu") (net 1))
 (segment (start 146.4513 90.2171) (end 147.5652 89.1032) (width 0.2) (layer "F.Cu") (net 1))
 (segment (start 146.4513 94.6826) (end 146.4513 90.2171) (width 0.2) (layer "F.Cu") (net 1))
 (segment (start 147.5652 89.1032) (end 152.5929 89.1032) (width 0.2) (layer "F.Cu") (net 1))
 (segment (start 141.6824 95.8923) (end 141.6824 95.9542) (width 0.2) (layer "F.Cu") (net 1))
 (segment (start 154.3827 86.214) (end 152.5929 88.0038) (width 0.2) (layer "F.Cu") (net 1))
 (via (at 152.5929 89.1032) (size 0.6) (drill 0.3) (layers "F.Cu" "B.Cu") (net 1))
 (segment (start 152.146 89.5501) (end 152.5929 89.1032) (width 0.2) (layer "B.Cu") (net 1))
 (segment (start 152.146 90.3732) (end 152.146 89.5501) (width 0.2) (layer "B.Cu") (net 1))
 (segment (start 155.683 83.118) (end 150.2345 83.118) (width 0.2) (layer "F.Cu") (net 17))
 (via (at 150.2345 83.118) (size 0.6) (drill 0.3) (layers "F.Cu" "B.Cu") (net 17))
 (segment (start 148.1595 83.118) (end 150.2345 83.118) (width 0.2) (layer "B.Cu") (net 17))
 (segment (start 148.1503 83.1088) (end 148.1595 83.118) (width 0.2) (layer "B.Cu") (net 17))
 (segment (start 147.35 83.1088) (end 148.1503 83.1088) (width 0.2) (layer "B.Cu") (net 17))
 (segment (start 142.0826 85.5794) (end 143.5896 84.0724) (width 0.2) (layer "F.Cu") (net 6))
 (segment (start 142.0826 86.0099) (end 142.0826 85.5794) (width 0.2) (layer "F.Cu") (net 6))
 (segment (start 140.5965 87.496) (end 142.0826 86.0099) (width 0.2) (layer "F.Cu") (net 6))
 (segment (start 144.8652 84.0724) (end 145.4098 84.617) (width 0.2) (layer "F.Cu") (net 6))
 (segment (start 139.435 87.496) (end 140.5965 87.496) (width 0.2) (layer "F.Cu") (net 6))
 (segment (start 143.5896 84.0724) (end 144.8652 84.0724) (width 0.2) (layer "F.Cu") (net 6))
 (via (at 145.4098 84.617) (size 0.6) (drill 0.3) (layers "F.Cu" "B.Cu") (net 6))
 (segment (start 145.8677 84.1591) (end 145.4098 84.617) (width 0.2) (layer "B.Cu") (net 6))
 (segment (start 146.05 83.1088) (end 146.05 84.1591) (width 0.2) (layer "B.Cu") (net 6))
 (segment (start 146.05 84.1591) (end 145.8677 84.1591) (width 0.2) (layer "B.Cu") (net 6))
 (segment (start 143.383 86.214) (end 144.6833 86.214) (width 0.2) (layer "F.Cu") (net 14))
 (segment (start 144.6833 86.214) (end 144.6833 84.7512) (width 0.2) (layer "F.Cu") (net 14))
 (segment (start 144.6833 84.7512) (end 144.6049 84.6728) (width 0.2) (layer "F.Cu") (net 14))
 (via (at 144.6049 84.6728) (size 0.6) (drill 0.3) (layers "F.Cu" "B.Cu") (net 14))
 (segment (start 144.75 83.1088) (end 144.75 84.1591) (width 0.2) (layer "B.Cu") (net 14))
 (segment (start 144.6049 84.3042) (end 144.75 84.1591) (width 0.2) (layer "B.Cu") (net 14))
 (segment (start 144.6049 84.6728) (end 144.6049 84.3042) (width 0.2) (layer "B.Cu") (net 14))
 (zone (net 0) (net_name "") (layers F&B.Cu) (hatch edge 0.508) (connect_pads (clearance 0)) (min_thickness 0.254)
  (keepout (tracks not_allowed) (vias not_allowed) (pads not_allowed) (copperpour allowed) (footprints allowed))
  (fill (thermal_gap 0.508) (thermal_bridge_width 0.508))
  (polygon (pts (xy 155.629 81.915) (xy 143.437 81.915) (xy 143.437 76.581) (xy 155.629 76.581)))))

